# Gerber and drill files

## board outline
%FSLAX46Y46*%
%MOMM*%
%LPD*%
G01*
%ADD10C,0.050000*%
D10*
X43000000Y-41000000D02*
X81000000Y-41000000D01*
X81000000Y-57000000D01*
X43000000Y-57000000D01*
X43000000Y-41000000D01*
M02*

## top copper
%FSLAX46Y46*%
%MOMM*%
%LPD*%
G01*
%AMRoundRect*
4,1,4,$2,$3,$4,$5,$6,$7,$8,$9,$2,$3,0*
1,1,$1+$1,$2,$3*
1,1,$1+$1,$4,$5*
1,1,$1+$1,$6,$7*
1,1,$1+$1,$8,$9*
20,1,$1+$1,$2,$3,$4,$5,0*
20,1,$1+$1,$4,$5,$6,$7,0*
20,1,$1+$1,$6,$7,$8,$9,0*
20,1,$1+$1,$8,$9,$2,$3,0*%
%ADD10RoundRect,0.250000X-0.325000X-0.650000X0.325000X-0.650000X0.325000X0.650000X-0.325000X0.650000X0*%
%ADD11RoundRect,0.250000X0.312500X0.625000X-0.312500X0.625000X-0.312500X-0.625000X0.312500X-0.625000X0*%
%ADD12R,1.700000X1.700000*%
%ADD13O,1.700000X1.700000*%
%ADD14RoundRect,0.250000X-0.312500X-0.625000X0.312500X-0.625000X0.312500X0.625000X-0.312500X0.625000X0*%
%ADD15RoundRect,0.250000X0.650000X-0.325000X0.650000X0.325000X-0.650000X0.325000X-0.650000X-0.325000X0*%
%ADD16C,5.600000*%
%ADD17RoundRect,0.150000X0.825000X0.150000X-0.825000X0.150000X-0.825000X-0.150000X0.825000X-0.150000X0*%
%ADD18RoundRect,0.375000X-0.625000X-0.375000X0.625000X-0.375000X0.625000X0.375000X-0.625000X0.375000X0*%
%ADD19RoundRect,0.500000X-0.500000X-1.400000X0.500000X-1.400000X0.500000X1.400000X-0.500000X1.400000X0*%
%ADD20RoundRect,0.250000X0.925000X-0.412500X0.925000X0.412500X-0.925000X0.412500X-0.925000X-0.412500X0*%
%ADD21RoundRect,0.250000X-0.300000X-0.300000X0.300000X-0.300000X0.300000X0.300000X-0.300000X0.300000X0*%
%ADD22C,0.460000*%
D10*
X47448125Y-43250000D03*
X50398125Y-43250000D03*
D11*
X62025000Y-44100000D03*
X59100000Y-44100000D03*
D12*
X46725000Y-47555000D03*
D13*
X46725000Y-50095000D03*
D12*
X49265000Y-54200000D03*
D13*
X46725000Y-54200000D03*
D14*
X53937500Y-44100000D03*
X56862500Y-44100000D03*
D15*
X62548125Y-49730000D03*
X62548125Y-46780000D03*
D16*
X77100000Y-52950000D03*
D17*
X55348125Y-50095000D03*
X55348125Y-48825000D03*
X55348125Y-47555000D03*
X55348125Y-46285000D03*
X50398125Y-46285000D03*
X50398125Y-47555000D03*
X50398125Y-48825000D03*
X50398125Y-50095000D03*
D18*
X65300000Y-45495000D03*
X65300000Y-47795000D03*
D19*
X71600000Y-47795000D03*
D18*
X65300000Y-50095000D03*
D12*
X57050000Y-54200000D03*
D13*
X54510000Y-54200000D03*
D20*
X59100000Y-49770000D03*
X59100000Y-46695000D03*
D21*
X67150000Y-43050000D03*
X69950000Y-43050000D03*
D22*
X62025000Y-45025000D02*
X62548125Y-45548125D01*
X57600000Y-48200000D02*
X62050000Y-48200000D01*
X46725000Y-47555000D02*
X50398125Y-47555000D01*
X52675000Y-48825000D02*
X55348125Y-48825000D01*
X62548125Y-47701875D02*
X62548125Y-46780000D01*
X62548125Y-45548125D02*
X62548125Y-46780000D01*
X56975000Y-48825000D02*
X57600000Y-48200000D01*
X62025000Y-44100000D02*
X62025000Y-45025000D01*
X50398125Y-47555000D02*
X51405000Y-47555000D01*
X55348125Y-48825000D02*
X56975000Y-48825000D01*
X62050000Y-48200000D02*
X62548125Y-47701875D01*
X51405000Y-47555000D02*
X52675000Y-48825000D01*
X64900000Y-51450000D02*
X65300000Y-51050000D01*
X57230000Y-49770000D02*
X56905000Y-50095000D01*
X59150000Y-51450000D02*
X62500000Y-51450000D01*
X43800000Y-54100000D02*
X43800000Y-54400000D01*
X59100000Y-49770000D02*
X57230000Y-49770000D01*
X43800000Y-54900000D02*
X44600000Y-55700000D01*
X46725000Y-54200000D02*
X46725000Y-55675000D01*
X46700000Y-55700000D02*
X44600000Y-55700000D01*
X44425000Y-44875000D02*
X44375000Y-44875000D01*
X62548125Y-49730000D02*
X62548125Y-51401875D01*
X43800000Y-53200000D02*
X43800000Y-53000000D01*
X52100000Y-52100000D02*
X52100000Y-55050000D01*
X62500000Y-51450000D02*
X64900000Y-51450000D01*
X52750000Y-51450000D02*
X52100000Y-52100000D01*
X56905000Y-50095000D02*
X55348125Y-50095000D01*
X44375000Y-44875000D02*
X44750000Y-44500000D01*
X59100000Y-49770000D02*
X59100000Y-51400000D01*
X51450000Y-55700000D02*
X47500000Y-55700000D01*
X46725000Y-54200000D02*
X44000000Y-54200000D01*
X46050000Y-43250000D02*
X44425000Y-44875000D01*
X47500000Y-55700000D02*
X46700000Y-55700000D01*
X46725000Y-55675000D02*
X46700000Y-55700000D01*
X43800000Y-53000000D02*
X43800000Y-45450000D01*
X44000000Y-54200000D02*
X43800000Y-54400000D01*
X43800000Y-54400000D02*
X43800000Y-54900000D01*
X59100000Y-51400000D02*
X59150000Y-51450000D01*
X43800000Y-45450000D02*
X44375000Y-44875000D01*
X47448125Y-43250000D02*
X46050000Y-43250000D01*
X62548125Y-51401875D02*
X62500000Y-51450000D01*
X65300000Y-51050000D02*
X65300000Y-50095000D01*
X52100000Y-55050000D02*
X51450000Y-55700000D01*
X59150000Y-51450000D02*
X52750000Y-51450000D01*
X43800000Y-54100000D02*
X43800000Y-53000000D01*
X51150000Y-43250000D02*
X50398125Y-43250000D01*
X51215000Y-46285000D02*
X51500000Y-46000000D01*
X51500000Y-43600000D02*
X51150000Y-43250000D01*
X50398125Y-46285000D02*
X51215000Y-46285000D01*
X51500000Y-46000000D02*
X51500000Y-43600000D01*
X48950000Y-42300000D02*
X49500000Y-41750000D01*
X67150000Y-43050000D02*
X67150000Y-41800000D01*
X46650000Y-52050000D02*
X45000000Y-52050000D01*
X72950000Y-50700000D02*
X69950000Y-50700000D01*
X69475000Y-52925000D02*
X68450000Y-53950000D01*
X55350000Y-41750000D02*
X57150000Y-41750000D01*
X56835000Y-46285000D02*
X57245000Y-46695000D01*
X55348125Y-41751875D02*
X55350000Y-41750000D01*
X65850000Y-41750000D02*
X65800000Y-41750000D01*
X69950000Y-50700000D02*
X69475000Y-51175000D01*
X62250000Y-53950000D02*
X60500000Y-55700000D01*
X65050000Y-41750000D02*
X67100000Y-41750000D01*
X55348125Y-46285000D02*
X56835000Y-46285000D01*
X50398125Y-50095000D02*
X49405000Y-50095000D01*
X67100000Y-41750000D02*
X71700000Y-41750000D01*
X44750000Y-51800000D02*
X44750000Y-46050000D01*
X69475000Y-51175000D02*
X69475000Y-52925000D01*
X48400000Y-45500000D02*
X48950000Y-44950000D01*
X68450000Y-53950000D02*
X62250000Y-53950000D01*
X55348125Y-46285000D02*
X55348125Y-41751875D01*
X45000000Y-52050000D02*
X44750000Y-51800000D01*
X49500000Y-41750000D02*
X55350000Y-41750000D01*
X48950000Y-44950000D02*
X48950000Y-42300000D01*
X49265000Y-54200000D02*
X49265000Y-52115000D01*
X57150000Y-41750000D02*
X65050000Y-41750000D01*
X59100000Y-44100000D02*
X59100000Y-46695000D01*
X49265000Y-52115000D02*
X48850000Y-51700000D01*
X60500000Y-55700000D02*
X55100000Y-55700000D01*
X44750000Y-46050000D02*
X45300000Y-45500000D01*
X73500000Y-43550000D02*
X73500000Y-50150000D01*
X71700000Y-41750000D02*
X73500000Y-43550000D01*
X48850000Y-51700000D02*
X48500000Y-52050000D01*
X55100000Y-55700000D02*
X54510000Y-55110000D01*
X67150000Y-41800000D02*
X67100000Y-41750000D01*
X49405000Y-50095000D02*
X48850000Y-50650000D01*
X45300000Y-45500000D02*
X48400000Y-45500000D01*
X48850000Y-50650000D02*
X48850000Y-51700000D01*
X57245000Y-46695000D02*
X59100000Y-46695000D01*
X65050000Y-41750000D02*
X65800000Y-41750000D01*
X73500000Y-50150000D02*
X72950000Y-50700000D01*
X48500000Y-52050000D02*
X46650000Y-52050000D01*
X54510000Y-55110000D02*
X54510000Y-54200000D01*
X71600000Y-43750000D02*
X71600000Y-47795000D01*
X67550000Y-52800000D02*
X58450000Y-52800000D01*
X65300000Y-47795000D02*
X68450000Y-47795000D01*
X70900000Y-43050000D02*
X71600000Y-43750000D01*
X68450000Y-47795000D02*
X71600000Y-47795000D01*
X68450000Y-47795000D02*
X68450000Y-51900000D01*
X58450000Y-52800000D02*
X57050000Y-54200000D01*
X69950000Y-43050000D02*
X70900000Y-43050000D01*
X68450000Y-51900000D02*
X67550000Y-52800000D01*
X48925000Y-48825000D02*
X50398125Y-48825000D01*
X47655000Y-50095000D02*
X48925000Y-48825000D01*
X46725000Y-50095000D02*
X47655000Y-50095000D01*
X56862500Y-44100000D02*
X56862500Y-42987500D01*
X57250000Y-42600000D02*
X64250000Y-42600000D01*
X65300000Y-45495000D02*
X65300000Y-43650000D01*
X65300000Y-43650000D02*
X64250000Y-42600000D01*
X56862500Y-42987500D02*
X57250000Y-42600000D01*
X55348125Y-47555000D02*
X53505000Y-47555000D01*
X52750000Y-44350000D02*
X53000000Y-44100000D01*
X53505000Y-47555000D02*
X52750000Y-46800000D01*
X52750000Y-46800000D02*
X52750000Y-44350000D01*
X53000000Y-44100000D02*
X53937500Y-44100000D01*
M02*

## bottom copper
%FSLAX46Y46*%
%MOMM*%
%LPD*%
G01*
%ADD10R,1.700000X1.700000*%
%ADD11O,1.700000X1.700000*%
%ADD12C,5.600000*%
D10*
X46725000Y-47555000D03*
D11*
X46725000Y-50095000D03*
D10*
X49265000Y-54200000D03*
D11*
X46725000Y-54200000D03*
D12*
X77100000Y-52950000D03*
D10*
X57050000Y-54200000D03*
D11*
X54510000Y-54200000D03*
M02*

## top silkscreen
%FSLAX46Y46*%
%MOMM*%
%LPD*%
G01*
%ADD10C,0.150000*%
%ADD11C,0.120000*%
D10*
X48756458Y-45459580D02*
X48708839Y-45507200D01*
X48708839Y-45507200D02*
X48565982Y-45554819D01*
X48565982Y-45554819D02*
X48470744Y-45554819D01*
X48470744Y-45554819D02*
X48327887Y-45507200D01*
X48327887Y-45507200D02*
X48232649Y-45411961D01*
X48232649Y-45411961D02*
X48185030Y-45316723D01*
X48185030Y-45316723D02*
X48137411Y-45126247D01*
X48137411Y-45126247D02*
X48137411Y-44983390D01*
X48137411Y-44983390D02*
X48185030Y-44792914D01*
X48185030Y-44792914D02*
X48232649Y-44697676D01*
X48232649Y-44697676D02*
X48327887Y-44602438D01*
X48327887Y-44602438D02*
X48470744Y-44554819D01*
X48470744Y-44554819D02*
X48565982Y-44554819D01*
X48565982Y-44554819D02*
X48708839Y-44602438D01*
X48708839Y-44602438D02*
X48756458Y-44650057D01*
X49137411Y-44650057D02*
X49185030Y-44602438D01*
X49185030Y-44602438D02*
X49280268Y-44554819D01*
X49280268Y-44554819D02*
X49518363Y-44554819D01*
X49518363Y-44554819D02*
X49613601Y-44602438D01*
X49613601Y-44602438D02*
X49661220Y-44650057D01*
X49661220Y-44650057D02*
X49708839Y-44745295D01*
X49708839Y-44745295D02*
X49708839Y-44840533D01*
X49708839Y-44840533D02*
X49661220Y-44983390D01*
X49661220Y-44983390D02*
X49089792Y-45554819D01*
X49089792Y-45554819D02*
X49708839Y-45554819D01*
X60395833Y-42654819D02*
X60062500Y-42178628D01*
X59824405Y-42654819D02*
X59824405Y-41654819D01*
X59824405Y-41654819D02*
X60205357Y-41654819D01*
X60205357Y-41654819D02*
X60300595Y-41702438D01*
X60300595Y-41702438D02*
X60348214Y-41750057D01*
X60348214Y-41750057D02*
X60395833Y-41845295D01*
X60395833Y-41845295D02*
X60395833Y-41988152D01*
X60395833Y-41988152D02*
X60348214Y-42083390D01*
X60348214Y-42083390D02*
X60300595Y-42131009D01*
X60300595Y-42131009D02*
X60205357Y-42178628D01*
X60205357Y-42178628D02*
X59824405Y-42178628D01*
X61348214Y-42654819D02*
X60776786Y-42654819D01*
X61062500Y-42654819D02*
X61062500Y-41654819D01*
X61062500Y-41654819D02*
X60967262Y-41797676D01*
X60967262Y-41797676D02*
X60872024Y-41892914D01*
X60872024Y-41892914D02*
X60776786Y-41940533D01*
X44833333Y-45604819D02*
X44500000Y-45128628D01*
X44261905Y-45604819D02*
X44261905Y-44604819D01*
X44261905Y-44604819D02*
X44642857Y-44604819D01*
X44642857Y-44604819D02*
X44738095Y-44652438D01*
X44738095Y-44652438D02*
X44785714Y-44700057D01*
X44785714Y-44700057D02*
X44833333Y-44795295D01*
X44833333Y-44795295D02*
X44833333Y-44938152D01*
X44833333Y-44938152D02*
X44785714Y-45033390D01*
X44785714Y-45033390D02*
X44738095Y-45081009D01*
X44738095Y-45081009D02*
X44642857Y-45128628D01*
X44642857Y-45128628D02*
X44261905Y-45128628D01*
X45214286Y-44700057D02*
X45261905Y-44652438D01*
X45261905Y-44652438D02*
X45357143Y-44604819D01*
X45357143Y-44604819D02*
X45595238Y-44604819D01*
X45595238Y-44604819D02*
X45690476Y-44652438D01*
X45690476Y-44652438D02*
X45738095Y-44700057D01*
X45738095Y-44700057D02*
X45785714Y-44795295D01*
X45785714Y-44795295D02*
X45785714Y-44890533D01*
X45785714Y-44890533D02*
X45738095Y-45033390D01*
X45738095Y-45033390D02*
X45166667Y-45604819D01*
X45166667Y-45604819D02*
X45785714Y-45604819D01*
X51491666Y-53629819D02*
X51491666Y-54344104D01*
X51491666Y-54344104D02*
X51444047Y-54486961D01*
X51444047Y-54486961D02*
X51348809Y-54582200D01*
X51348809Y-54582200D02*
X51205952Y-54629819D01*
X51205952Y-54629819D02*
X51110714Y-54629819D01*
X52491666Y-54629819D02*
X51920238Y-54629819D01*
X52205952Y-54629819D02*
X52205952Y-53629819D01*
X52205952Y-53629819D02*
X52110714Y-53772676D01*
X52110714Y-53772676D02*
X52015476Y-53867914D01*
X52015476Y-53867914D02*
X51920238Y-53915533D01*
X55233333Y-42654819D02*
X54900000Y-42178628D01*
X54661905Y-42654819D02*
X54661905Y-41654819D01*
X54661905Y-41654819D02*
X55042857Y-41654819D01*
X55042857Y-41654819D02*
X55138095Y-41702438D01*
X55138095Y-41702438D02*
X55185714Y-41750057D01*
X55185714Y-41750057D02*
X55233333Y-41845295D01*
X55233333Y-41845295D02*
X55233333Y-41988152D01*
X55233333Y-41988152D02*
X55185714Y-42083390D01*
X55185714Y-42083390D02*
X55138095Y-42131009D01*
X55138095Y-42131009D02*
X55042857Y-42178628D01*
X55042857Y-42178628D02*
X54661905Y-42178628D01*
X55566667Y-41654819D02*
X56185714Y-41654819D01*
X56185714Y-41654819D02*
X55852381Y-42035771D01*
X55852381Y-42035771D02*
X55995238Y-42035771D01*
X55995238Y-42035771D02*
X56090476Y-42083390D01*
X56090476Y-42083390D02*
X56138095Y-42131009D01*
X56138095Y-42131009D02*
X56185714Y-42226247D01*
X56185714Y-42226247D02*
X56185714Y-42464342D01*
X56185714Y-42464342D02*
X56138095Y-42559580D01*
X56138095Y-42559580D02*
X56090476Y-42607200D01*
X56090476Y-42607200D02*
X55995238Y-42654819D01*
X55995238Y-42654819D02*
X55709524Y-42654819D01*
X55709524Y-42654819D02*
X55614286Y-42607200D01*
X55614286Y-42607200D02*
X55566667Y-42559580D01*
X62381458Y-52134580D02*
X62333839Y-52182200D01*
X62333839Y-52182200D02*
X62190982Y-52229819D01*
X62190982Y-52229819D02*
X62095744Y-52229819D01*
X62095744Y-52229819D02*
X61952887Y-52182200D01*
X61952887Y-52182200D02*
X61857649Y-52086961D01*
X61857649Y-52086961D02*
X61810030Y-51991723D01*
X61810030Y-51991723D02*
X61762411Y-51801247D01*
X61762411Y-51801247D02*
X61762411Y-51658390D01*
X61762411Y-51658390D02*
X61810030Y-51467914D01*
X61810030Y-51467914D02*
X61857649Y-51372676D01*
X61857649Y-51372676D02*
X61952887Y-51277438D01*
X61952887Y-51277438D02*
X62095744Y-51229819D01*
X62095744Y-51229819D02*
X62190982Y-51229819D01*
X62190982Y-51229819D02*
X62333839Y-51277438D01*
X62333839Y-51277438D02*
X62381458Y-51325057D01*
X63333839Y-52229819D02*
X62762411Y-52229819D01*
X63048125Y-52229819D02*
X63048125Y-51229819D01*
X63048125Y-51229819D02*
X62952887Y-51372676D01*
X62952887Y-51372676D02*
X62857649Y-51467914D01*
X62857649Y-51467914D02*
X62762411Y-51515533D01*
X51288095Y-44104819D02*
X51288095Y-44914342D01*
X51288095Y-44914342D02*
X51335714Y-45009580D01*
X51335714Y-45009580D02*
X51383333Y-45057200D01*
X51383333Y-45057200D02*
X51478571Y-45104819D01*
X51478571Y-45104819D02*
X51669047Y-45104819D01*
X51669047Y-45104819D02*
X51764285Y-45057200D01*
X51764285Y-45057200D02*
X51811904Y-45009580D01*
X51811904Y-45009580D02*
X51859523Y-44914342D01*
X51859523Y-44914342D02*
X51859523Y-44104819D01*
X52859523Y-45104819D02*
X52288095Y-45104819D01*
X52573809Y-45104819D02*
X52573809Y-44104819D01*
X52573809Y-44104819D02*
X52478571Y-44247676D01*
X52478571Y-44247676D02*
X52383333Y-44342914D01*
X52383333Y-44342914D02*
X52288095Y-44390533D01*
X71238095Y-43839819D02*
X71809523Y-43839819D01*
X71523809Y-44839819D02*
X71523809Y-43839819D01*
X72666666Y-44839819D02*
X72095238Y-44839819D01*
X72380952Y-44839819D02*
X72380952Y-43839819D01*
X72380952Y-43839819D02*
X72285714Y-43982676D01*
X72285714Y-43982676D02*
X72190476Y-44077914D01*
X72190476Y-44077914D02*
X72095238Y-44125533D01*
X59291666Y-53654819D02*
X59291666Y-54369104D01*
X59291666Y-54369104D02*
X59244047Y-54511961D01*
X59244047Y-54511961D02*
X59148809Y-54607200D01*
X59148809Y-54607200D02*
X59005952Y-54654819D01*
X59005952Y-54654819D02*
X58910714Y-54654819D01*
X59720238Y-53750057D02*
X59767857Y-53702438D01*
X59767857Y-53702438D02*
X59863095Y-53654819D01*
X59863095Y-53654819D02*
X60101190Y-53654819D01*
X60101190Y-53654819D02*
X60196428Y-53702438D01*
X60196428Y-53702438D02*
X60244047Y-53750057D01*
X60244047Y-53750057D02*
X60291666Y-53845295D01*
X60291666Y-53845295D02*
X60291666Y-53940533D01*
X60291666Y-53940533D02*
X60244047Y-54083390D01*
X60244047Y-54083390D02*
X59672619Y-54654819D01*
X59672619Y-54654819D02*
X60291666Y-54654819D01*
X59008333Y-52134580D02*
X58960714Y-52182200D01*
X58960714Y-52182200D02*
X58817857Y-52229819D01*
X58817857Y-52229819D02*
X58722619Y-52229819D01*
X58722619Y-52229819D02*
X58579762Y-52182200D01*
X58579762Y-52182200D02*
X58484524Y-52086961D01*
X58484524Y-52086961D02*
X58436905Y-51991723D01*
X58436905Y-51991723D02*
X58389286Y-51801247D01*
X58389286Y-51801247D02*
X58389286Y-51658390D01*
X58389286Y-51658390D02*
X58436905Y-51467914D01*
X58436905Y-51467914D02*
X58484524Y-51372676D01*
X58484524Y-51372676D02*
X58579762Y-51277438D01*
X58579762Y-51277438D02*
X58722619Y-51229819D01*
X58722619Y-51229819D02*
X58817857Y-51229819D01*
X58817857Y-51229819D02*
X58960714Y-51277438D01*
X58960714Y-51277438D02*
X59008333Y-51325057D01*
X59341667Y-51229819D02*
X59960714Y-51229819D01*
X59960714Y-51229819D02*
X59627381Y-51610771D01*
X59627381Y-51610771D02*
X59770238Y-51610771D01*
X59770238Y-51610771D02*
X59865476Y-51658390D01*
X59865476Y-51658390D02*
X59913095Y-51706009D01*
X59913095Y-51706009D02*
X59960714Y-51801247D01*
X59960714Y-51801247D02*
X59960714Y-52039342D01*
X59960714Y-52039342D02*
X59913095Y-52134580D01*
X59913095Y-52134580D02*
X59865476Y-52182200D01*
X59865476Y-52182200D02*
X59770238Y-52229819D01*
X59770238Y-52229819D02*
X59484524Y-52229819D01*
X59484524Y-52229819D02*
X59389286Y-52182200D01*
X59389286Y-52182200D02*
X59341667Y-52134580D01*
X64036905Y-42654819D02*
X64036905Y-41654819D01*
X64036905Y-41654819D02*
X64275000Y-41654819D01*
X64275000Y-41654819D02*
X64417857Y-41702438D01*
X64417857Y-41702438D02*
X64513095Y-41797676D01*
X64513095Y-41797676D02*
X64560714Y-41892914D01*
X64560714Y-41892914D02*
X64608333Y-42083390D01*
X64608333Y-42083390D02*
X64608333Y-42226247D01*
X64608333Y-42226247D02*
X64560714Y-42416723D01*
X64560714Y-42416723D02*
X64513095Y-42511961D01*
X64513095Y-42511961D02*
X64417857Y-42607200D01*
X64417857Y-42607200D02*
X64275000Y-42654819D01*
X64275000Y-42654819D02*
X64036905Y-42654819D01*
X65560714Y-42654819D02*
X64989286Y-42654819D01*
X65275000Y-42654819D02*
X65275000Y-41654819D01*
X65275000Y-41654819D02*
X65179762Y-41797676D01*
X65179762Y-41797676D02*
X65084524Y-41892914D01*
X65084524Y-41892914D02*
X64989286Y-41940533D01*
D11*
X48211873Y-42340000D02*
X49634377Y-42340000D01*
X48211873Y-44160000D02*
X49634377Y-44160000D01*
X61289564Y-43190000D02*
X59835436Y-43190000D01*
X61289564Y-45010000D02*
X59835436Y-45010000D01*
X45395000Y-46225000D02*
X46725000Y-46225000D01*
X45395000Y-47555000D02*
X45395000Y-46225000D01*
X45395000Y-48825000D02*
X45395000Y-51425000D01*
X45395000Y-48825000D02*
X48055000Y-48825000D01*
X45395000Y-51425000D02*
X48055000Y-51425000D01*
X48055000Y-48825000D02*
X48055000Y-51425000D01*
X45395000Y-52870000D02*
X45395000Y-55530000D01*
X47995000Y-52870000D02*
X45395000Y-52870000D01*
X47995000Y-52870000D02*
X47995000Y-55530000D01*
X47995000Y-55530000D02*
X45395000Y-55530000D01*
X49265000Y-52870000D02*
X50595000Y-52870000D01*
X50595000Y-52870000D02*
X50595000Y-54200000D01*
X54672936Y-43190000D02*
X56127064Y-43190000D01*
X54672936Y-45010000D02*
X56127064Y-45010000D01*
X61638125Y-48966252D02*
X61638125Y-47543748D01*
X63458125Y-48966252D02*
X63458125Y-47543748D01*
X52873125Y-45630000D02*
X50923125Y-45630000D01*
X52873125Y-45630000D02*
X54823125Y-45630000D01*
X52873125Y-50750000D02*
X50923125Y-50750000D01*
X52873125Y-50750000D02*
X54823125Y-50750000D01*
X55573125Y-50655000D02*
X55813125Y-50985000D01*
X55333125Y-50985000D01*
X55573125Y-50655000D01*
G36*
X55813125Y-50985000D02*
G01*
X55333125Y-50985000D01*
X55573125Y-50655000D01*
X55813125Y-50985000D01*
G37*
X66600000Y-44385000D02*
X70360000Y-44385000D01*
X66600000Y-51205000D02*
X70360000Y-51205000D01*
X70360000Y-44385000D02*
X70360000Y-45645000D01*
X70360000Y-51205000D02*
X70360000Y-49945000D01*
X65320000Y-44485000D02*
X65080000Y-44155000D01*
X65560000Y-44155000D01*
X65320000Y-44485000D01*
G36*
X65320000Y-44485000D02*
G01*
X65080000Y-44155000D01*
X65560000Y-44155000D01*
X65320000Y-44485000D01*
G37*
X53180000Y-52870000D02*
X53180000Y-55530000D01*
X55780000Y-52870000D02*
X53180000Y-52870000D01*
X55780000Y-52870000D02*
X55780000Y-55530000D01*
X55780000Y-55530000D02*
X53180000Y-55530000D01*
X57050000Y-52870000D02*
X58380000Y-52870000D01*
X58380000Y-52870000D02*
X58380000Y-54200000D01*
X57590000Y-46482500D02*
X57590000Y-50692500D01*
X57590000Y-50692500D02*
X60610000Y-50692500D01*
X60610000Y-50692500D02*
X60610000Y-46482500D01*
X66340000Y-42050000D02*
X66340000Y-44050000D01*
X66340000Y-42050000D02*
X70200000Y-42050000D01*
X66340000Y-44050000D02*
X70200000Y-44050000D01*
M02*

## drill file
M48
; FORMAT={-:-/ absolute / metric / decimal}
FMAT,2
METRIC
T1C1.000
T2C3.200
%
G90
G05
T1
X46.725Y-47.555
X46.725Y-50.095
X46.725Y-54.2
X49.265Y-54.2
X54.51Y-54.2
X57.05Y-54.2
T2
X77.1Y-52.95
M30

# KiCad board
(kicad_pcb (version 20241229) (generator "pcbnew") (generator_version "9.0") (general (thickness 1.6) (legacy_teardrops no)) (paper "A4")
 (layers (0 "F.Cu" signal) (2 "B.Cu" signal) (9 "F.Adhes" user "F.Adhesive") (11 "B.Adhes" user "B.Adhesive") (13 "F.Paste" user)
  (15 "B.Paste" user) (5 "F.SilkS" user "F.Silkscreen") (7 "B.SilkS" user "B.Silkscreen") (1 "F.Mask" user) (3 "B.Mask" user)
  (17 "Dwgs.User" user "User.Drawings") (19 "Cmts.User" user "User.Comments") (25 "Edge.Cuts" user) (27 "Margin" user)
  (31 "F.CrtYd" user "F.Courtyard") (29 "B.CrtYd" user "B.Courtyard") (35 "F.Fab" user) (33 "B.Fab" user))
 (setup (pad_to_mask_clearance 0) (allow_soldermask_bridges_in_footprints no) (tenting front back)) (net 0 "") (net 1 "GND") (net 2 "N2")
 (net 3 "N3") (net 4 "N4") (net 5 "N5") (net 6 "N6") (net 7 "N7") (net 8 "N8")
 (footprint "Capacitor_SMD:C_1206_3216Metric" (layer "F.Cu") (at 48.923125 43.25)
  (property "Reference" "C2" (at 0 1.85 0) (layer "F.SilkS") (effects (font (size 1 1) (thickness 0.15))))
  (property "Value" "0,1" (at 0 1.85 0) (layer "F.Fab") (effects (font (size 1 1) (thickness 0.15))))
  (fp_line (start -0.711252 -0.91) (end 0.711252 -0.91) (stroke (width 0.12) (type solid)) (layer "F.SilkS"))
  (fp_line (start -0.711252 0.91) (end 0.711252 0.91) (stroke (width 0.12) (type solid)) (layer "F.SilkS"))
  (pad "1" smd roundrect (at -1.475 0) (size 1.15 1.8) (layers "F.Cu" "F.Mask" "F.Paste") (roundrect_rratio 0.217391) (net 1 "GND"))
  (pad "2" smd roundrect (at 1.475 0) (size 1.15 1.8) (layers "F.Cu" "F.Mask" "F.Paste") (roundrect_rratio 0.217391) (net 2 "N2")))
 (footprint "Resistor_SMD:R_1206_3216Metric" (layer "F.Cu") (at 60.5625 44.1 180)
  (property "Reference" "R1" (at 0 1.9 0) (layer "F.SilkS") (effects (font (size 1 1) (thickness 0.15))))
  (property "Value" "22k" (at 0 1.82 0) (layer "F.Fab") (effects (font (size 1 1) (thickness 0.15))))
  (fp_line (start -0.727064 0.91) (end 0.727064 0.91) (stroke (width 0.12) (type solid)) (layer "F.SilkS"))
  (fp_line (start -0.727064 -0.91) (end 0.727064 -0.91) (stroke (width 0.12) (type solid)) (layer "F.SilkS"))
  (pad "1" smd roundrect (at -1.4625 0 180) (size 1.125 1.75) (layers "F.Cu" "F.Mask" "F.Paste") (roundrect_rratio 0.222222) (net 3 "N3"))
  (pad "2" smd roundrect (at 1.4625 0 180) (size 1.125 1.75) (layers "F.Cu" "F.Mask" "F.Paste") (roundrect_rratio 0.222222) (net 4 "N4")))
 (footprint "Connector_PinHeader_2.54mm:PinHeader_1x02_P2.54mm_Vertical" (layer "F.Cu") (at 46.725 47.555)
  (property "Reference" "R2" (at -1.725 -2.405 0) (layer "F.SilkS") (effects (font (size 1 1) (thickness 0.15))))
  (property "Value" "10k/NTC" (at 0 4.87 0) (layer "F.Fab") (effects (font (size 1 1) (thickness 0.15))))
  (fp_line (start -1.33 -1.33) (end 0 -1.33) (stroke (width 0.12) (type solid)) (layer "F.SilkS"))
  (fp_line (start -1.33 0) (end -1.33 -1.33) (stroke (width 0.12) (type solid)) (layer "F.SilkS"))
  (fp_line (start -1.33 1.27) (end -1.33 3.87) (stroke (width 0.12) (type solid)) (layer "F.SilkS"))
  (fp_line (start -1.33 1.27) (end 1.33 1.27) (stroke (width 0.12) (type solid)) (layer "F.SilkS"))
  (fp_line (start -1.33 3.87) (end 1.33 3.87) (stroke (width 0.12) (type solid)) (layer "F.SilkS"))
  (fp_line (start 1.33 1.27) (end 1.33 3.87) (stroke (width 0.12) (type solid)) (layer "F.SilkS"))
  (pad "1" thru_hole rect (at 0 0) (size 1.7 1.7) (drill 1) (layers "*.Cu" "*.Mask") (remove_unused_layers no) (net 3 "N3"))
  (pad "2" thru_hole oval (at 0 2.54) (size 1.7 1.7) (drill 1) (layers "*.Cu" "*.Mask") (remove_unused_layers no) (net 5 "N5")))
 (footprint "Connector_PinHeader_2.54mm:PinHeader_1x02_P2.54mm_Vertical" (layer "F.Cu") (at 49.265 54.2 -90)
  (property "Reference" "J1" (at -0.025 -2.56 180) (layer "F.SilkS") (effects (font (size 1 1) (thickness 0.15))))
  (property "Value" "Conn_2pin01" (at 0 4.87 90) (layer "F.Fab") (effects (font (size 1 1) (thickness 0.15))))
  (fp_line (start -1.33 3.87) (end 1.33 3.87) (stroke (width 0.12) (type solid)) (layer "F.SilkS"))
  (fp_line (start -1.33 1.27) (end -1.33 3.87) (stroke (width 0.12) (type solid)) (layer "F.SilkS"))
  (fp_line (start -1.33 1.27) (end 1.33 1.27) (stroke (width 0.12) (type solid)) (layer "F.SilkS"))
  (fp_line (start 1.33 1.27) (end 1.33 3.87) (stroke (width 0.12) (type solid)) (layer "F.SilkS"))
  (fp_line (start -1.33 0) (end -1.33 -1.33) (stroke (width 0.12) (type solid)) (layer "F.SilkS"))
  (fp_line (start -1.33 -1.33) (end 0 -1.33) (stroke (width 0.12) (type solid)) (layer "F.SilkS"))
  (pad "1" thru_hole rect (at 0 0 270) (size 1.7 1.7) (drill 1) (layers "*.Cu" "*.Mask") (remove_unused_layers no) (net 4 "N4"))
  (pad "2" thru_hole oval (at 0 2.54 270) (size 1.7 1.7) (drill 1) (layers "*.Cu" "*.Mask") (remove_unused_layers no) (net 1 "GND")))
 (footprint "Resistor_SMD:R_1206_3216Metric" (layer "F.Cu") (at 55.4 44.1)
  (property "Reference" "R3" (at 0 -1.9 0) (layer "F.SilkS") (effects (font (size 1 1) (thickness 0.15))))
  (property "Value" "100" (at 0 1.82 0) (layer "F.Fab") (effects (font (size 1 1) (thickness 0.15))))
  (fp_line (start -0.727064 -0.91) (end 0.727064 -0.91) (stroke (width 0.12) (type solid)) (layer "F.SilkS"))
  (fp_line (start -0.727064 0.91) (end 0.727064 0.91) (stroke (width 0.12) (type solid)) (layer "F.SilkS"))
  (pad "1" smd roundrect (at -1.4625 0) (size 1.125 1.75) (layers "F.Cu" "F.Mask" "F.Paste") (roundrect_rratio 0.222222) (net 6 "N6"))
  (pad "2" smd roundrect (at 1.4625 0) (size 1.125 1.75) (layers "F.Cu" "F.Mask" "F.Paste") (roundrect_rratio 0.222222) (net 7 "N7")))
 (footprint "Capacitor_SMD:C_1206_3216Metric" (layer "F.Cu") (at 62.548125 48.255 90)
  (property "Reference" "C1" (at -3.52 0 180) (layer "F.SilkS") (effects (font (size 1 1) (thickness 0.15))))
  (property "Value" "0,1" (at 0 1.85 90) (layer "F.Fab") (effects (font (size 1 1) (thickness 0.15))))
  (fp_line (start -0.711252 -0.91) (end 0.711252 -0.91) (stroke (width 0.12) (type solid)) (layer "F.SilkS"))
  (fp_line (start -0.711252 0.91) (end 0.711252 0.91) (stroke (width 0.12) (type solid)) (layer "F.SilkS"))
  (pad "1" smd roundrect (at -1.475 0 90) (size 1.15 1.8) (layers "F.Cu" "F.Mask" "F.Paste") (roundrect_rratio 0.217391) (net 1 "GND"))
  (pad "2" smd roundrect (at 1.475 0 90) (size 1.15 1.8) (layers "F.Cu" "F.Mask" "F.Paste") (roundrect_rratio 0.217391) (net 3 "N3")))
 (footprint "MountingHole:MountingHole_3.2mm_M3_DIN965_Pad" (layer "F.Cu") (at 77.1 52.95)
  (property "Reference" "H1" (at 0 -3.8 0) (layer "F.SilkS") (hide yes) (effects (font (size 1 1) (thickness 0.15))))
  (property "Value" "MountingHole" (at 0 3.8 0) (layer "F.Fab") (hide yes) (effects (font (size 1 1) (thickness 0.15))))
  (pad "1" thru_hole circle (at 0 0) (size 5.6 5.6) (drill 3.2) (layers "*.Cu" "*.Mask") (remove_unused_layers no)))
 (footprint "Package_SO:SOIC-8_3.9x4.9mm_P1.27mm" (layer "F.Cu") (at 52.873125 48.19 180)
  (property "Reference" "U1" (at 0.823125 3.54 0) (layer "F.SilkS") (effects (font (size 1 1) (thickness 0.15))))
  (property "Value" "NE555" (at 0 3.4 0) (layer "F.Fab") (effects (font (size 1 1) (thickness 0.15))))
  (fp_line (start 0 2.56) (end 1.95 2.56) (stroke (width 0.12) (type solid)) (layer "F.SilkS"))
  (fp_line (start 0 2.56) (end -1.95 2.56) (stroke (width 0.12) (type solid)) (layer "F.SilkS"))
  (fp_line (start 0 -2.56) (end 1.95 -2.56) (stroke (width 0.12) (type solid)) (layer "F.SilkS"))
  (fp_line (start 0 -2.56) (end -1.95 -2.56) (stroke (width 0.12) (type solid)) (layer "F.SilkS"))
  (fp_poly
   (pts (xy -2.7 -2.465) (xy -2.94 -2.795) (xy -2.46 -2.795) (xy -2.7 -2.465)) (stroke (width 0.12) (type solid)) (fill yes)
   (layer "F.SilkS"))
  (pad "1" smd roundrect (at -2.475 -1.905 180) (size 1.95 0.6) (layers "F.Cu" "F.Mask" "F.Paste") (roundrect_rratio 0.25) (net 1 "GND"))
  (pad "2" smd roundrect (at -2.475 -0.635 180) (size 1.95 0.6) (layers "F.Cu" "F.Mask" "F.Paste") (roundrect_rratio 0.25) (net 3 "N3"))
  (pad "3" smd roundrect (at -2.475 0.635 180) (size 1.95 0.6) (layers "F.Cu" "F.Mask" "F.Paste") (roundrect_rratio 0.25) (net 6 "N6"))
  (pad "4" smd roundrect (at -2.475 1.905 180) (size 1.95 0.6) (layers "F.Cu" "F.Mask" "F.Paste") (roundrect_rratio 0.25) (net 4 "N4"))
  (pad "5" smd roundrect (at 2.475 1.905 180) (size 1.95 0.6) (layers "F.Cu" "F.Mask" "F.Paste") (roundrect_rratio 0.25) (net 2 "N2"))
  (pad "6" smd roundrect (at 2.475 0.635 180) (size 1.95 0.6) (layers "F.Cu" "F.Mask" "F.Paste") (roundrect_rratio 0.25) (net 3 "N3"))
  (pad "7" smd roundrect (at 2.475 -0.635 180) (size 1.95 0.6) (layers "F.Cu" "F.Mask" "F.Paste") (roundrect_rratio 0.25) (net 5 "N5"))
  (pad "8" smd roundrect (at 2.475 -1.905 180) (size 1.95 0.6) (layers "F.Cu" "F.Mask" "F.Paste") (roundrect_rratio 0.25) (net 4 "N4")))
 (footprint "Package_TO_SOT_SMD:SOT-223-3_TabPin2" (layer "F.Cu") (at 68.45 47.795)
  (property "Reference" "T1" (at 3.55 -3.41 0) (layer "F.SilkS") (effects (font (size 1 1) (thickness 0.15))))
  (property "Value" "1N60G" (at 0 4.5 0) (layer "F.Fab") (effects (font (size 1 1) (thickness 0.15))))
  (fp_line (start -1.85 -3.41) (end 1.91 -3.41) (stroke (width 0.12) (type solid)) (layer "F.SilkS"))
  (fp_line (start -1.85 3.41) (end 1.91 3.41) (stroke (width 0.12) (type solid)) (layer "F.SilkS"))
  (fp_line (start 1.91 -3.41) (end 1.91 -2.15) (stroke (width 0.12) (type solid)) (layer "F.SilkS"))
  (fp_line (start 1.91 3.41) (end 1.91 2.15) (stroke (width 0.12) (type solid)) (layer "F.SilkS"))
  (fp_poly
   (pts (xy -3.13 -3.31) (xy -3.37 -3.64) (xy -2.89 -3.64) (xy -3.13 -3.31)) (stroke (width 0.12) (type solid)) (fill yes) (layer "F.SilkS"))
  (pad "1" smd roundrect (at -3.15 -2.3) (size 2 1.5) (layers "F.Cu" "F.Mask" "F.Paste") (roundrect_rratio 0.25) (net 7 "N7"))
  (pad "2" smd roundrect (at -3.15 0) (size 2 1.5) (layers "F.Cu" "F.Mask" "F.Paste") (roundrect_rratio 0.25) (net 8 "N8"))
  (pad "2" smd roundrect (at 3.15 0) (size 2 3.8) (layers "F.Cu" "F.Mask" "F.Paste") (roundrect_rratio 0.25) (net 8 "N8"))
  (pad "3" smd roundrect (at -3.15 2.3) (size 2 1.5) (layers "F.Cu" "F.Mask" "F.Paste") (roundrect_rratio 0.25) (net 1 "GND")))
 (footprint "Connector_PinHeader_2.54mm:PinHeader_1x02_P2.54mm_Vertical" (layer "F.Cu") (at 57.05 54.2 -90)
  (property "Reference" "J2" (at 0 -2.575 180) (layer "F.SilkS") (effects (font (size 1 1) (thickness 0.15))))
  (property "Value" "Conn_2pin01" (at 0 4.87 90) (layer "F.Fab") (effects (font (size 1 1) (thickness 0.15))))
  (fp_line (start -1.33 3.87) (end 1.33 3.87) (stroke (width 0.12) (type solid)) (layer "F.SilkS"))
  (fp_line (start -1.33 1.27) (end -1.33 3.87) (stroke (width 0.12) (type solid)) (layer "F.SilkS"))
  (fp_line (start -1.33 1.27) (end 1.33 1.27) (stroke (width 0.12) (type solid)) (layer "F.SilkS"))
  (fp_line (start 1.33 1.27) (end 1.33 3.87) (stroke (width 0.12) (type solid)) (layer "F.SilkS"))
  (fp_line (start -1.33 0) (end -1.33 -1.33) (stroke (width 0.12) (type solid)) (layer "F.SilkS"))
  (fp_line (start -1.33 -1.33) (end 0 -1.33) (stroke (width 0.12) (type solid)) (layer "F.SilkS"))
  (pad "1" thru_hole rect (at 0 0 270) (size 1.7 1.7) (drill 1) (layers "*.Cu" "*.Mask") (remove_unused_layers no) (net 8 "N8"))
  (pad "2" thru_hole oval (at 0 2.54 270) (size 1.7 1.7) (drill 1) (layers "*.Cu" "*.Mask") (remove_unused_layers no) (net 4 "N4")))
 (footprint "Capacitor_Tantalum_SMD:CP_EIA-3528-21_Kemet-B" (layer "F.Cu") (at 59.1 48.2325 90)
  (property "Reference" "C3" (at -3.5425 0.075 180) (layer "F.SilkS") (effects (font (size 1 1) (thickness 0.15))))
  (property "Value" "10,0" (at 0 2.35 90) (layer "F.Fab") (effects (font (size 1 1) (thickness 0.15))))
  (fp_line (start 1.75 -1.51) (end -2.46 -1.51) (stroke (width 0.12) (type solid)) (layer "F.SilkS"))
  (fp_line (start -2.46 -1.51) (end -2.46 1.51) (stroke (width 0.12) (type solid)) (layer "F.SilkS"))
  (fp_line (start -2.46 1.51) (end 1.75 1.51) (stroke (width 0.12) (type solid)) (layer "F.SilkS"))
  (pad "1" smd roundrect (at -1.5375 0 90) (size 1.325 2.35) (layers "F.Cu" "F.Mask" "F.Paste") (roundrect_rratio 0.188679) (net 1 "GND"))
  (pad "2" smd roundrect (at 1.5375 0 90) (size 1.325 2.35) (layers "F.Cu" "F.Mask" "F.Paste") (roundrect_rratio 0.188679) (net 4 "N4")))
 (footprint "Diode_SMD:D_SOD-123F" (layer "F.Cu") (at 68.55 43.05)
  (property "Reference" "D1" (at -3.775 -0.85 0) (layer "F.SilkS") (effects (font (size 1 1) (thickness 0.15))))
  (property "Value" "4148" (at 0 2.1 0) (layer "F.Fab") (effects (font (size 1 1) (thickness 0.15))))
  (fp_line (start -2.21 -1) (end -2.21 1) (stroke (width 0.12) (type solid)) (layer "F.SilkS"))
  (fp_line (start -2.21 -1) (end 1.65 -1) (stroke (width 0.12) (type solid)) (layer "F.SilkS"))
  (fp_line (start -2.21 1) (end 1.65 1) (stroke (width 0.12) (type solid)) (layer "F.SilkS"))
  (pad "1" smd roundrect (at -1.4 0) (size 1.1 1.1) (layers "F.Cu" "F.Mask" "F.Paste") (roundrect_rratio 0.2272727273) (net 4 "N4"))
  (pad "2" smd roundrect (at 1.4 0) (size 1.1 1.1) (layers "F.Cu" "F.Mask" "F.Paste") (roundrect_rratio 0.2272727273) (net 8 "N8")))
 (gr_rect (start 43 41) (end 81 57) (stroke (width 0.05) (type default)) (fill no) (layer "Edge.Cuts"))
 (segment (start 62.025 45.025) (end 62.548125 45.548125) (width 0.46) (layer "F.Cu") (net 3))
 (segment (start 57.6 48.2) (end 62.05 48.2) (width 0.46) (layer "F.Cu") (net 3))
 (segment (start 46.725 47.555) (end 50.398125 47.555) (width 0.46) (layer "F.Cu") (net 3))
 (segment (start 52.675 48.825) (end 55.348125 48.825) (width 0.46) (layer "F.Cu") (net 3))
 (segment (start 62.548125 47.701875) (end 62.548125 46.78) (width 0.46) (layer "F.Cu") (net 3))
 (segment (start 62.548125 45.548125) (end 62.548125 46.78) (width 0.46) (layer "F.Cu") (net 3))
 (segment (start 56.975 48.825) (end 57.6 48.2) (width 0.46) (layer "F.Cu") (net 3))
 (segment (start 62.025 44.1) (end 62.025 45.025) (width 0.46) (layer "F.Cu") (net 3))
 (segment (start 50.398125 47.555) (end 51.405 47.555) (width 0.46) (layer "F.Cu") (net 3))
 (segment (start 55.348125 48.825) (end 56.975 48.825) (width 0.46) (layer "F.Cu") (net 3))
 (segment (start 62.05 48.2) (end 62.548125 47.701875) (width 0.46) (layer "F.Cu") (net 3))
 (segment (start 51.405 47.555) (end 52.675 48.825) (width 0.46) (layer "F.Cu") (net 3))
 (segment (start 64.9 51.45) (end 65.3 51.05) (width 0.46) (layer "F.Cu") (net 1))
 (segment (start 57.23 49.77) (end 56.905 50.095) (width 0.46) (layer "F.Cu") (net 1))
 (segment (start 59.15 51.45) (end 62.5 51.45) (width 0.46) (layer "F.Cu") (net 1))
 (segment (start 43.8 54.1) (end 43.8 54.4) (width 0.46) (layer "F.Cu") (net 1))
 (segment (start 59.1 49.77) (end 57.23 49.77) (width 0.46) (layer "F.Cu") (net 1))
 (segment (start 43.8 54.9) (end 44.6 55.7) (width 0.46) (layer "F.Cu") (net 1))
 (segment (start 46.725 54.2) (end 46.725 55.675) (width 0.46) (layer "F.Cu") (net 1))
 (segment (start 46.7 55.7) (end 44.6 55.7) (width 0.46) (layer "F.Cu") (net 1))
 (segment (start 44.425 44.875) (end 44.375 44.875) (width 0.46) (layer "F.Cu") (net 1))
 (segment (start 62.548125 49.73) (end 62.548125 51.401875) (width 0.46) (layer "F.Cu") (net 1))
 (segment (start 43.8 53.2) (end 43.8 53) (width 0.46) (layer "F.Cu") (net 1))
 (segment (start 52.1 52.1) (end 52.1 55.05) (width 0.46) (layer "F.Cu") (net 1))
 (segment (start 62.5 51.45) (end 64.9 51.45) (width 0.46) (layer "F.Cu") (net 1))
 (segment (start 52.75 51.45) (end 52.1 52.1) (width 0.46) (layer "F.Cu") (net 1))
 (segment (start 56.905 50.095) (end 55.348125 50.095) (width 0.46) (layer "F.Cu") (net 1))
 (segment (start 44.375 44.875) (end 44.75 44.5) (width 0.46) (layer "F.Cu") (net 1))
 (segment (start 59.1 49.77) (end 59.1 51.4) (width 0.46) (layer "F.Cu") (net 1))
 (segment (start 51.45 55.7) (end 47.5 55.7) (width 0.46) (layer "F.Cu") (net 1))
 (segment (start 46.725 54.2) (end 44 54.2) (width 0.46) (layer "F.Cu") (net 1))
 (segment (start 46.05 43.25) (end 44.425 44.875) (width 0.46) (layer "F.Cu") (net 1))
 (segment (start 47.5 55.7) (end 46.7 55.7) (width 0.46) (layer "F.Cu") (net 1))
 (segment (start 46.725 55.675) (end 46.7 55.7) (width 0.46) (layer "F.Cu") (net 1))
 (segment (start 43.8 53) (end 43.8 45.45) (width 0.46) (layer "F.Cu") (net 1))
 (segment (start 44 54.2) (end 43.8 54.4) (width 0.46) (layer "F.Cu") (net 1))
 (segment (start 43.8 54.4) (end 43.8 54.9) (width 0.46) (layer "F.Cu") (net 1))
 (segment (start 59.1 51.4) (end 59.15 51.45) (width 0.46) (layer "F.Cu") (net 1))
 (segment (start 43.8 45.45) (end 44.375 44.875) (width 0.46) (layer "F.Cu") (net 1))
 (segment (start 47.448125 43.25) (end 46.05 43.25) (width 0.46) (layer "F.Cu") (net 1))
 (segment (start 62.548125 51.401875) (end 62.5 51.45) (width 0.46) (layer "F.Cu") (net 1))
 (segment (start 65.3 51.05) (end 65.3 50.095) (width 0.46) (layer "F.Cu") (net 1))
 (segment (start 52.1 55.05) (end 51.45 55.7) (width 0.46) (layer "F.Cu") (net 1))
 (segment (start 59.15 51.45) (end 52.75 51.45) (width 0.46) (layer "F.Cu") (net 1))
 (segment (start 43.8 54.1) (end 43.8 53) (width 0.46) (layer "F.Cu") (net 1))
 (segment (start 51.15 43.25) (end 50.398125 43.25) (width 0.46) (layer "F.Cu") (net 2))
 (segment (start 51.215 46.285) (end 51.5 46) (width 0.46) (layer "F.Cu") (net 2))
 (segment (start 51.5 43.6) (end 51.15 43.25) (width 0.46) (layer "F.Cu") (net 2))
 (segment (start 50.398125 46.285) (end 51.215 46.285) (width 0.46) (layer "F.Cu") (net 2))
 (segment (start 51.5 46) (end 51.5 43.6) (width 0.46) (layer "F.Cu") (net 2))
 (segment (start 48.95 42.3) (end 49.5 41.75) (width 0.46) (layer "F.Cu") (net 4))
 (segment (start 67.15 43.05) (end 67.15 41.8) (width 0.46) (layer "F.Cu") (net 4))
 (segment (start 46.65 52.05) (end 45 52.05) (width 0.46) (layer "F.Cu") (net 4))
 (segment (start 72.95 50.7) (end 69.95 50.7) (width 0.46) (layer "F.Cu") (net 4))
 (segment (start 69.475 52.925) (end 68.45 53.95) (width 0.46) (layer "F.Cu") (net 4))
 (segment (start 55.35 41.75) (end 57.15 41.75) (width 0.46) (layer "F.Cu") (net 4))
 (segment (start 56.835 46.285) (end 57.245 46.695) (width 0.46) (layer "F.Cu") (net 4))
 (segment (start 55.348125 41.751875) (end 55.35 41.75) (width 0.46) (layer "F.Cu") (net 4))
 (segment (start 65.85 41.75) (end 65.8 41.75) (width 0.46) (layer "F.Cu") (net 4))
 (segment (start 69.95 50.7) (end 69.475 51.175) (width 0.46) (layer "F.Cu") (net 4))
 (segment (start 62.25 53.95) (end 60.5 55.7) (width 0.46) (layer "F.Cu") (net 4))
 (segment (start 65.05 41.75) (end 67.1 41.75) (width 0.46) (layer "F.Cu") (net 4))
 (segment (start 55.348125 46.285) (end 56.835 46.285) (width 0.46) (layer "F.Cu") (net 4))
 (segment (start 50.398125 50.095) (end 49.405 50.095) (width 0.46) (layer "F.Cu") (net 4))
 (segment (start 67.1 41.75) (end 71.7 41.75) (width 0.46) (layer "F.Cu") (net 4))
 (segment (start 44.75 51.8) (end 44.75 46.05) (width 0.46) (layer "F.Cu") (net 4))
 (segment (start 69.475 51.175) (end 69.475 52.925) (width 0.46) (layer "F.Cu") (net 4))
 (segment (start 48.4 45.5) (end 48.95 44.95) (width 0.46) (layer "F.Cu") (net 4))
 (segment (start 68.45 53.95) (end 62.25 53.95) (width 0.46) (layer "F.Cu") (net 4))
 (segment (start 55.348125 46.285) (end 55.348125 41.751875) (width 0.46) (layer "F.Cu") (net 4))
 (segment (start 45 52.05) (end 44.75 51.8) (width 0.46) (layer "F.Cu") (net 4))
 (segment (start 49.5 41.75) (end 55.35 41.75) (width 0.46) (layer "F.Cu") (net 4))
 (segment (start 48.95 44.95) (end 48.95 42.3) (width 0.46) (layer "F.Cu") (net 4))
 (segment (start 49.265 54.2) (end 49.265 52.115) (width 0.46) (layer "F.Cu") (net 4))
 (segment (start 57.15 41.75) (end 65.05 41.75) (width 0.46) (layer "F.Cu") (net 4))
 (segment (start 59.1 44.1) (end 59.1 46.695) (width 0.46) (layer "F.Cu") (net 4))
 (segment (start 49.265 52.115) (end 48.85 51.7) (width 0.46) (layer "F.Cu") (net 4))
 (segment (start 60.5 55.7) (end 55.1 55.7) (width 0.46) (layer "F.Cu") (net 4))
 (segment (start 44.75 46.05) (end 45.3 45.5) (width 0.46) (layer "F.Cu") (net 4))
 (segment (start 73.5 43.55) (end 73.5 50.15) (width 0.46) (layer "F.Cu") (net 4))
 (segment (start 71.7 41.75) (end 73.5 43.55) (width 0.46) (layer "F.Cu") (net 4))
 (segment (start 48.85 51.7) (end 48.5 52.05) (width 0.46) (layer "F.Cu") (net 4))
 (segment (start 55.1 55.7) (end 54.51 55.11) (width 0.46) (layer "F.Cu") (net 4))
 (segment (start 67.15 41.8) (end 67.1 41.75) (width 0.46) (layer "F.Cu") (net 4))
 (segment (start 49.405 50.095) (end 48.85 50.65) (width 0.46) (layer "F.Cu") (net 4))
 (segment (start 45.3 45.5) (end 48.4 45.5) (width 0.46) (layer "F.Cu") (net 4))
 (segment (start 48.85 50.65) (end 48.85 51.7) (width 0.46) (layer "F.Cu") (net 4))
 (segment (start 57.245 46.695) (end 59.1 46.695) (width 0.46) (layer "F.Cu") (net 4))
 (segment (start 65.05 41.75) (end 65.8 41.75) (width 0.46) (layer "F.Cu") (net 4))
 (segment (start 73.5 50.15) (end 72.95 50.7) (width 0.46) (layer "F.Cu") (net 4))
 (segment (start 48.5 52.05) (end 46.65 52.05) (width 0.46) (layer "F.Cu") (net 4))
 (segment (start 54.51 55.11) (end 54.51 54.2) (width 0.46) (layer "F.Cu") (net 4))
 (segment (start 71.6 43.75) (end 71.6 47.795) (width 0.46) (layer "F.Cu") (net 8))
 (segment (start 67.55 52.8) (end 58.45 52.8) (width 0.46) (layer "F.Cu") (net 8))
 (segment (start 65.3 47.795) (end 68.45 47.795) (width 0.46) (layer "F.Cu") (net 8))
 (segment (start 70.9 43.05) (end 71.6 43.75) (width 0.46) (layer "F.Cu") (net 8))
 (segment (start 68.45 47.795) (end 71.6 47.795) (width 0.46) (layer "F.Cu") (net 8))
 (segment (start 68.45 47.795) (end 68.45 51.9) (width 0.46) (layer "F.Cu") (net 8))
 (segment (start 58.45 52.8) (end 57.05 54.2) (width 0.46) (layer "F.Cu") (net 8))
 (segment (start 69.95 43.05) (end 70.9 43.05) (width 0.46) (layer "F.Cu") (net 8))
 (segment (start 68.45 51.9) (end 67.55 52.8) (width 0.46) (layer "F.Cu") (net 8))
 (segment (start 48.925 48.825) (end 50.398125 48.825) (width 0.46) (layer "F.Cu") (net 5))
 (segment (start 47.655 50.095) (end 48.925 48.825) (width 0.46) (layer "F.Cu") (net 5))
 (segment (start 46.725 50.095) (end 47.655 50.095) (width 0.46) (layer "F.Cu") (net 5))
 (segment (start 56.8625 44.1) (end 56.8625 42.9875) (width 0.46) (layer "F.Cu") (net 7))
 (segment (start 57.25 42.6) (end 64.25 42.6) (width 0.46) (layer "F.Cu") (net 7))
 (segment (start 65.3 45.495) (end 65.3 43.65) (width 0.46) (layer "F.Cu") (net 7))
 (segment (start 65.3 43.65) (end 64.25 42.6) (width 0.46) (layer "F.Cu") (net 7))
 (segment (start 56.8625 42.9875) (end 57.25 42.6) (width 0.46) (layer "F.Cu") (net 7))
 (segment (start 55.348125 47.555) (end 53.505 47.555) (width 0.46) (layer "F.Cu") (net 6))
 (segment (start 52.75 44.35) (end 53 44.1) (width 0.46) (layer "F.Cu") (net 6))
 (segment (start 53.505 47.555) (end 52.75 46.8) (width 0.46) (layer "F.Cu") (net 6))
 (segment (start 52.75 46.8) (end 52.75 44.35) (width 0.46) (layer "F.Cu") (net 6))
 (segment (start 53 44.1) (end 53.9375 44.1) (width 0.46) (layer "F.Cu") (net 6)))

